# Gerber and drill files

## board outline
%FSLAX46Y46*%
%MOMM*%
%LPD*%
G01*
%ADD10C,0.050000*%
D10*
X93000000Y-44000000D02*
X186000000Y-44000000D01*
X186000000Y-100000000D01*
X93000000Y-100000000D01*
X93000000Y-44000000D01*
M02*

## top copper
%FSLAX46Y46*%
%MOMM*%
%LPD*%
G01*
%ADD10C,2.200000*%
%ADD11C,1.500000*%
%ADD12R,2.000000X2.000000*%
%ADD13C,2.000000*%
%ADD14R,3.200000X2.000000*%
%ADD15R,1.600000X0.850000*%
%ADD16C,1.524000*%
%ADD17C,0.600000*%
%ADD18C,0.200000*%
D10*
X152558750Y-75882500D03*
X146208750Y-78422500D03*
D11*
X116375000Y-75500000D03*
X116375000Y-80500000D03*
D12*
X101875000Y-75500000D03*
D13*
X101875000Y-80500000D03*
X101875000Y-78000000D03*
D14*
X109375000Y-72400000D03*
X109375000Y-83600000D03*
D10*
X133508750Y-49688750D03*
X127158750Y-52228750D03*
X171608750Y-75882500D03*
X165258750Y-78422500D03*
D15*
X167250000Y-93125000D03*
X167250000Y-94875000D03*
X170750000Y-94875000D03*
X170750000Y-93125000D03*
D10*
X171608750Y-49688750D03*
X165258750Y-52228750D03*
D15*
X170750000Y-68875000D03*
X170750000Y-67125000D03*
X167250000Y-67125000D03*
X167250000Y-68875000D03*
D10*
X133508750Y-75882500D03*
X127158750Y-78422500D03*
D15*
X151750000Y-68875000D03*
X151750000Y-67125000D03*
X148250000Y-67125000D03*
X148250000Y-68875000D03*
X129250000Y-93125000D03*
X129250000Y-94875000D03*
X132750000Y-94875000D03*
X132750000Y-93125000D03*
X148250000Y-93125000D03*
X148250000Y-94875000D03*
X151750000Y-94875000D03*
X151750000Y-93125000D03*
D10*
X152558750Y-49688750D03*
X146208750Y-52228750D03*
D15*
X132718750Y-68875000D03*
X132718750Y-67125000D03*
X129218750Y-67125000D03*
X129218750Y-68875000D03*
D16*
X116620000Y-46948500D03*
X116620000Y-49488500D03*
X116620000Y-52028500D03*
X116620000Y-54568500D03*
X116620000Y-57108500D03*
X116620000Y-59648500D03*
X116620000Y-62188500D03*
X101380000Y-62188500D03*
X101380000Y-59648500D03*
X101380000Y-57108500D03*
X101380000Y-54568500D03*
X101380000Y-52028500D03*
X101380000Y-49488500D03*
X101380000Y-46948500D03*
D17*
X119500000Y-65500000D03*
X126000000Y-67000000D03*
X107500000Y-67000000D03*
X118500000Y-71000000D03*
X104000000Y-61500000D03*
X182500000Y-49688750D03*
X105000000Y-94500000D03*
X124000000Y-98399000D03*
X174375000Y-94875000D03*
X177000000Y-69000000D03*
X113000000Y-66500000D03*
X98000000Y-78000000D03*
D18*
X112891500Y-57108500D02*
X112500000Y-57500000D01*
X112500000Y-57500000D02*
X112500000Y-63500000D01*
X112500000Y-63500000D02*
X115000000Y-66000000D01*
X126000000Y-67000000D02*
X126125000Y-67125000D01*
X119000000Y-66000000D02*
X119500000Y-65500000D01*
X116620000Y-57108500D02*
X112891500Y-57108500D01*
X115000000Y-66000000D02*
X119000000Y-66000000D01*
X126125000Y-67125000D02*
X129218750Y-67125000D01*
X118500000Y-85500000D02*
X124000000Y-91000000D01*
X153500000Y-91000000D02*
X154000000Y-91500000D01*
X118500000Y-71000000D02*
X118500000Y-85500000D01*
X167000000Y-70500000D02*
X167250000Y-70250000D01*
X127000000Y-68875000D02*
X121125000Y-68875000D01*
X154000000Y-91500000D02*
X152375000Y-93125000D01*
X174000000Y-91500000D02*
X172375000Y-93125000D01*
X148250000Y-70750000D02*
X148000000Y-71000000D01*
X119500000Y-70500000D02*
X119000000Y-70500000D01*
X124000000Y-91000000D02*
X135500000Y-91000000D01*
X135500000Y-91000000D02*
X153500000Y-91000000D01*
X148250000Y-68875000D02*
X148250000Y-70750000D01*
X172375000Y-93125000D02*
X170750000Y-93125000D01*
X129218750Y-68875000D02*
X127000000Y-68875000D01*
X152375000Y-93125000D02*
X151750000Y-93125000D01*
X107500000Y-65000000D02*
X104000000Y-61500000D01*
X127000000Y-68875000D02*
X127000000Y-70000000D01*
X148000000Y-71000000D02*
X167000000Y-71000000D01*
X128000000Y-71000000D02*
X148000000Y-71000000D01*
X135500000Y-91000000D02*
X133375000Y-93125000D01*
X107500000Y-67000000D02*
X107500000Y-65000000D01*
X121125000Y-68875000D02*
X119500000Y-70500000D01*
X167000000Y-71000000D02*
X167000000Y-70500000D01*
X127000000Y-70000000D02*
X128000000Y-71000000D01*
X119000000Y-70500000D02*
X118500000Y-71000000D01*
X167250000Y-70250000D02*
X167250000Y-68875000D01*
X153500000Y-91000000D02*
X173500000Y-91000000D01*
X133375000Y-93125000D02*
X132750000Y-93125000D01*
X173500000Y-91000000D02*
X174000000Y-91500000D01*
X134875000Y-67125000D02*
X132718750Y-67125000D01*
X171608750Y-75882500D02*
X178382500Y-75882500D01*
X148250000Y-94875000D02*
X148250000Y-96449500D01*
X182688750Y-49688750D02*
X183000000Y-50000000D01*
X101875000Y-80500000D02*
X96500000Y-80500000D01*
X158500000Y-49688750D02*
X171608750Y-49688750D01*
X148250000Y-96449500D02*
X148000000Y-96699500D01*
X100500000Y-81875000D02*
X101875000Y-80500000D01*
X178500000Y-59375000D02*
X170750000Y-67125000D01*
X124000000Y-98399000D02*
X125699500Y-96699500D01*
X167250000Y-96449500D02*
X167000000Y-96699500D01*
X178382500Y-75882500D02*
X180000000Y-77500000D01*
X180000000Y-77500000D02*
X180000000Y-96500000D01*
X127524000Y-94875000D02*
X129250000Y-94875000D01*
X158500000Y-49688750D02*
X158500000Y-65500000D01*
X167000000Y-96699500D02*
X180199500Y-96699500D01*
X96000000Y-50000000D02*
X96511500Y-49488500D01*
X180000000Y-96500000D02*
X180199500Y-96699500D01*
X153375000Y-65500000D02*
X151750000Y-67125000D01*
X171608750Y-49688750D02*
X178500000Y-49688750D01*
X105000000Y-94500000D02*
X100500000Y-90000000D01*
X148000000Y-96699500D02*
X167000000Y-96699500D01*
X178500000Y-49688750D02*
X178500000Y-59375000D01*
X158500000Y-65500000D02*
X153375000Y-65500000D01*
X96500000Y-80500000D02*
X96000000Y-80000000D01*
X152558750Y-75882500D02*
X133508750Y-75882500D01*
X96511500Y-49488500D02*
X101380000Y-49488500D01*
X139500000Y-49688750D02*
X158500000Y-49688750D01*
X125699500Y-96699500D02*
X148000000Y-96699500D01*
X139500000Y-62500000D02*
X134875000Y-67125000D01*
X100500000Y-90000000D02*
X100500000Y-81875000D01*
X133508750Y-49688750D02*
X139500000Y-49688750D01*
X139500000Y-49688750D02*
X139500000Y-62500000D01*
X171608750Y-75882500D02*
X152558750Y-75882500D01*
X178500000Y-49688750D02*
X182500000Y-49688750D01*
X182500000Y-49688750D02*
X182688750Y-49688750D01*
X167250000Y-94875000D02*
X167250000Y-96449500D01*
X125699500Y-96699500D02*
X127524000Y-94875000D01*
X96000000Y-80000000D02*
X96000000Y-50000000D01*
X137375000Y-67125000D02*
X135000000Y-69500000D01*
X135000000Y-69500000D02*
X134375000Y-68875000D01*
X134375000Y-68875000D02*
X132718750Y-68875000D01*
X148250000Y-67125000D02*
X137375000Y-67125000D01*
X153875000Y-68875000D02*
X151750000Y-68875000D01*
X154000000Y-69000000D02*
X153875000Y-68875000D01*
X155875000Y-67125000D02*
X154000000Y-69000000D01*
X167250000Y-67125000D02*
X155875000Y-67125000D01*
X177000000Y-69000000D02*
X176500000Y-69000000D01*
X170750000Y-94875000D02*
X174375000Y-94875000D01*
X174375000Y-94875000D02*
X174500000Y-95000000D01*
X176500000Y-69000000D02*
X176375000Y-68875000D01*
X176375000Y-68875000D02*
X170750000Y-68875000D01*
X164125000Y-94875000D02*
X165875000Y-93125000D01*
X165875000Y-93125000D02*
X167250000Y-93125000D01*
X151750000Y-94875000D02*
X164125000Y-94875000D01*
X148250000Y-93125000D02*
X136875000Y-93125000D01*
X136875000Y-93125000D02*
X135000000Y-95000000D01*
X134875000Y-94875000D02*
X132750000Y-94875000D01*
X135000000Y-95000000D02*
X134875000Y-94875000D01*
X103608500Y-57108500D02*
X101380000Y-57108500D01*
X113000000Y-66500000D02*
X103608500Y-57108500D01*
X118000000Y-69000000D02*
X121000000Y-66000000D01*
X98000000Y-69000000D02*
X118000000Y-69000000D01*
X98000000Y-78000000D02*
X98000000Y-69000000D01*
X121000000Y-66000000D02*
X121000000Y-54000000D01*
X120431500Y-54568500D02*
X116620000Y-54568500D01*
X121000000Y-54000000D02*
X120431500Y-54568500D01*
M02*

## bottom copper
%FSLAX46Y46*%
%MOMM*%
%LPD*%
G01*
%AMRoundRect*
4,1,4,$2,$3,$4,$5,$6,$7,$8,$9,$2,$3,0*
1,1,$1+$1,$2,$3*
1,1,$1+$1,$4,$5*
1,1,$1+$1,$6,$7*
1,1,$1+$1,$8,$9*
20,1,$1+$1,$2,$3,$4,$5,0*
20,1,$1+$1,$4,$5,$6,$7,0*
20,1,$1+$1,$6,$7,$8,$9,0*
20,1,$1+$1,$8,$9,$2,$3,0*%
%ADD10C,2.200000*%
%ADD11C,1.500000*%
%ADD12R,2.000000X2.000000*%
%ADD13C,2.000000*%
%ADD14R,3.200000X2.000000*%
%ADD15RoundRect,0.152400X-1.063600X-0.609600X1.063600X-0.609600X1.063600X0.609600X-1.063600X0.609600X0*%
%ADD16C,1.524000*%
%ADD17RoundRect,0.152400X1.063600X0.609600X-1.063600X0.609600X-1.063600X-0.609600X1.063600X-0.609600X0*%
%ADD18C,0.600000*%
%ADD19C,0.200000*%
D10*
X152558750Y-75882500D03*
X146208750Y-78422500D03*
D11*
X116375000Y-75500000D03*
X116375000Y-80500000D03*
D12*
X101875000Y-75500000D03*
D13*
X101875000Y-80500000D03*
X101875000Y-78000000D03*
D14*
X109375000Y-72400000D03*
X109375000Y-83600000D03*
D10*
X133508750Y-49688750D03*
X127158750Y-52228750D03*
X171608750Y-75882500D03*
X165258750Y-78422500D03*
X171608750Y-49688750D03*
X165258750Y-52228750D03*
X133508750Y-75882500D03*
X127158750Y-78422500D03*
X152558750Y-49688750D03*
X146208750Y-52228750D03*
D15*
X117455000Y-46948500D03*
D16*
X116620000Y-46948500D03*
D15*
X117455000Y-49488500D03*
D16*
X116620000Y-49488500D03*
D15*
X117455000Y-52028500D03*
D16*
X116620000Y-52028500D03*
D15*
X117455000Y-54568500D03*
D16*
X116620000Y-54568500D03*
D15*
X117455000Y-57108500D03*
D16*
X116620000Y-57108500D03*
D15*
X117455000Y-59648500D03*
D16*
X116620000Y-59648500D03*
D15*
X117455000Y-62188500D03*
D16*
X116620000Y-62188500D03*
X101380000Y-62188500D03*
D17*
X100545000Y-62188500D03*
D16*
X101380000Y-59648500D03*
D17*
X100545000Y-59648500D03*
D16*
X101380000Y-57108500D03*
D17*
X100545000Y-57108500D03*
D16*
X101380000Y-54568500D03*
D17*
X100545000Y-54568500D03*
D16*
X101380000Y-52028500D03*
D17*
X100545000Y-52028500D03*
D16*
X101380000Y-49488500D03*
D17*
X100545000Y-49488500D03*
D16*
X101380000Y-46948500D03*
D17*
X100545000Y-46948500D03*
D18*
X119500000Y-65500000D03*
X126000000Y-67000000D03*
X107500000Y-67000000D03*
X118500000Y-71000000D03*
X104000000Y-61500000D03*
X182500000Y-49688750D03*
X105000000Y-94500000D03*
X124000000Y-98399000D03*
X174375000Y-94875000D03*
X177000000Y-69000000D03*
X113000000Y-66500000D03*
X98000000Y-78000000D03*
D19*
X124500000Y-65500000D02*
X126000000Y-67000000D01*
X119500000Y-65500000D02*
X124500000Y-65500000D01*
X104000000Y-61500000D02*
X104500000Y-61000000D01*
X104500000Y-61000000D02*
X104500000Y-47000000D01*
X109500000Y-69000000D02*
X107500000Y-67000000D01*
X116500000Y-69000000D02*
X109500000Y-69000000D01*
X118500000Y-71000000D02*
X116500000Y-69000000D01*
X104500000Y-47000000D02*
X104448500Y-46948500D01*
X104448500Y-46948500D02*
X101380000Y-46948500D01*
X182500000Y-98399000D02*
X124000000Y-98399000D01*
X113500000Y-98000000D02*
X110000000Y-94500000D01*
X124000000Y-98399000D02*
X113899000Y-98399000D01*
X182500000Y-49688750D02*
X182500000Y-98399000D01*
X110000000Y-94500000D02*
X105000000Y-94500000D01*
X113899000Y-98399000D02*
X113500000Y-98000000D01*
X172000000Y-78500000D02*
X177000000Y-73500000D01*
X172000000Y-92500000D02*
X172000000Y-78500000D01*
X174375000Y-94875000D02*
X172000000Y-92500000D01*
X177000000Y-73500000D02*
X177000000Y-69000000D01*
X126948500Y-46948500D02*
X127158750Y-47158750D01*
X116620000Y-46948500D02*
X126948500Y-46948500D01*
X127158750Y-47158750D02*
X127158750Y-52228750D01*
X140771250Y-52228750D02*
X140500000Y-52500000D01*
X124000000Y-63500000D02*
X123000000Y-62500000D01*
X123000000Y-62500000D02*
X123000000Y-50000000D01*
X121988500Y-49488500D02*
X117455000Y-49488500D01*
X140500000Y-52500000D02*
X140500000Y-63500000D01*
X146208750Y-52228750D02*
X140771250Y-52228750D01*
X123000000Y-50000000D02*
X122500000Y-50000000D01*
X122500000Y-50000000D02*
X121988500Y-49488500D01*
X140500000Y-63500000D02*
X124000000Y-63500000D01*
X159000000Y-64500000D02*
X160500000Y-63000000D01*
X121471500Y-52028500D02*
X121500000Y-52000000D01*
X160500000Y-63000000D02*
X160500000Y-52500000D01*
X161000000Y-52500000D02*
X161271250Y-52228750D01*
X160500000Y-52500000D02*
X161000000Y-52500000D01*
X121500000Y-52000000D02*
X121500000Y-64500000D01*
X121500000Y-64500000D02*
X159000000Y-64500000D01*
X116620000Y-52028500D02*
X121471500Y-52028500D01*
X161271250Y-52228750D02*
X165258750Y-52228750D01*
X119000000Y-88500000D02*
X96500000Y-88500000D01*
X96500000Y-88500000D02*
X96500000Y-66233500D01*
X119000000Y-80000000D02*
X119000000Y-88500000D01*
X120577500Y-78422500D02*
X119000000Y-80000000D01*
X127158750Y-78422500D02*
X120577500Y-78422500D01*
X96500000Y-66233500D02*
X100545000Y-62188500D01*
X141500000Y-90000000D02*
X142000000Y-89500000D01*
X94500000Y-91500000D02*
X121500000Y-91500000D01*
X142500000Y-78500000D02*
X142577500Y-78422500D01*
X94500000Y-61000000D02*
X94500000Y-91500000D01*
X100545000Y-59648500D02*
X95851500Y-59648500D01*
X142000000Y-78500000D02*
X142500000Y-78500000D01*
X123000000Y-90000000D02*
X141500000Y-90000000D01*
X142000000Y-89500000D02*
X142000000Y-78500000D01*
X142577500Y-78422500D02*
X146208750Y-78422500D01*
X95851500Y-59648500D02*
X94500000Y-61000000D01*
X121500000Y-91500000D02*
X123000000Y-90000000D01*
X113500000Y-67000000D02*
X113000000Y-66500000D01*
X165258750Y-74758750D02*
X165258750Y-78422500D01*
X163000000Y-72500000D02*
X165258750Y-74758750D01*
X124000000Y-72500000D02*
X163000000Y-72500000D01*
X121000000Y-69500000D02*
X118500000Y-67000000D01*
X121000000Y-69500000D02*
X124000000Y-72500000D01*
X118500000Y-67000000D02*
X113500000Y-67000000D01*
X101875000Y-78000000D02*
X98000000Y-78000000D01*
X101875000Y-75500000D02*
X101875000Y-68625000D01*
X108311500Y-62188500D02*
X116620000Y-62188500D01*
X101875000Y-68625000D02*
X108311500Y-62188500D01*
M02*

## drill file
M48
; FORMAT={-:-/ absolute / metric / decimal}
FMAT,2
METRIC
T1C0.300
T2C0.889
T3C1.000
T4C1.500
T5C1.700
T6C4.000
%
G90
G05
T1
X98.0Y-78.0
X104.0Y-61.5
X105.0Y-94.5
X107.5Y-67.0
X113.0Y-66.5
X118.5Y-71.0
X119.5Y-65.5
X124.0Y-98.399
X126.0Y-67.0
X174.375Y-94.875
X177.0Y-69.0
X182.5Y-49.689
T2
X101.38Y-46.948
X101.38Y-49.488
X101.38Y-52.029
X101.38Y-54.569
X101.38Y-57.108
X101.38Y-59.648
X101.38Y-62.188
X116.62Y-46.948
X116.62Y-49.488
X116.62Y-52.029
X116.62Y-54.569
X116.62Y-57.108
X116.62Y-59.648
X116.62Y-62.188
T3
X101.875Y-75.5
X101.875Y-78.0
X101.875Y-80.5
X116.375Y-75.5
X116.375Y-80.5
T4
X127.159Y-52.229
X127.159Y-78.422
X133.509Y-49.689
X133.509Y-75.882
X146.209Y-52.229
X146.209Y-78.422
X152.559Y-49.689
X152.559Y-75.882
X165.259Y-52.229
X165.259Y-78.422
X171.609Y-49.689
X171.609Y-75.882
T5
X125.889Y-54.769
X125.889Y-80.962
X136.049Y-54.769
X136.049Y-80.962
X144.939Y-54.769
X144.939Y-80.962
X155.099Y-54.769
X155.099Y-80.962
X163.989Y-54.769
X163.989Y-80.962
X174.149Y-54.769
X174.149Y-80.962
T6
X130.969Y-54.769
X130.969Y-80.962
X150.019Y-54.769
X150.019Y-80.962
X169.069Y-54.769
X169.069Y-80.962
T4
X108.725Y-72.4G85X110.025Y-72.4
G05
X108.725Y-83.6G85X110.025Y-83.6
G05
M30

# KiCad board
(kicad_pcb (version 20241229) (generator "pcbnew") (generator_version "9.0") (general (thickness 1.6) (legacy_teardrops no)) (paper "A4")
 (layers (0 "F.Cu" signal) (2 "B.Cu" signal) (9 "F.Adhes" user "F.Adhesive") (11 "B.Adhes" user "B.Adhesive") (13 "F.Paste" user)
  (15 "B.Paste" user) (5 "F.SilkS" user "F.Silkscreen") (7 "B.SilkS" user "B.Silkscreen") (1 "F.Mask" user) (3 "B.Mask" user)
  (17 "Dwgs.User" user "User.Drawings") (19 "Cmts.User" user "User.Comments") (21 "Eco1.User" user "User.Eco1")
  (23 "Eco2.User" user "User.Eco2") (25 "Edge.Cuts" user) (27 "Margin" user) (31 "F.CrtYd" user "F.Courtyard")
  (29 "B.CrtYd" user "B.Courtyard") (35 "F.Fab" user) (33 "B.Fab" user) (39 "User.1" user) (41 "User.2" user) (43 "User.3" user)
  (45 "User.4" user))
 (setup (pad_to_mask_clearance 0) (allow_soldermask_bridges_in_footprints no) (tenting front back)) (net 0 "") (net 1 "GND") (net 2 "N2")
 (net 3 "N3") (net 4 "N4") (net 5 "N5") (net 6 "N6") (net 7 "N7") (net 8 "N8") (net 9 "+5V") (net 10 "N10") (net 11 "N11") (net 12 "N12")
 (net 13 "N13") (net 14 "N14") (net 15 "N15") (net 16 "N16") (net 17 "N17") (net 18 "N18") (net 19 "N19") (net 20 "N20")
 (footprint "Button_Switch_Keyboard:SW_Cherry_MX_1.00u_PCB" (layer "F.Cu") (at 152.55875 75.8825)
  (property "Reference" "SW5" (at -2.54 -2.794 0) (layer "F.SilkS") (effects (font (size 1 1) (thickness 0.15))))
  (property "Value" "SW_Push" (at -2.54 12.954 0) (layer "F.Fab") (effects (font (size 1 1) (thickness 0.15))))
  (pad "" np_thru_hole circle (at -7.62 5.08) (size 1.7 1.7) (drill 1.7) (layers "*.Cu" "*.Mask"))
  (pad "" np_thru_hole circle (at -2.54 5.08) (size 4 4) (drill 4) (layers "*.Cu" "*.Mask"))
  (pad "" np_thru_hole circle (at 2.54 5.08) (size 1.7 1.7) (drill 1.7) (layers "*.Cu" "*.Mask"))
  (pad "1" thru_hole circle (at 0 0) (size 2.2 2.2) (drill 1.5) (layers "*.Cu" "*.Mask") (remove_unused_layers no) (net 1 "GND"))
  (pad "2" thru_hole circle (at -6.35 2.54) (size 2.2 2.2) (drill 1.5) (layers "*.Cu" "*.Mask") (remove_unused_layers no) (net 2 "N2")))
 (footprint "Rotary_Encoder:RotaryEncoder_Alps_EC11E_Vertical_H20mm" (layer "F.Cu") (at 101.875 75.5)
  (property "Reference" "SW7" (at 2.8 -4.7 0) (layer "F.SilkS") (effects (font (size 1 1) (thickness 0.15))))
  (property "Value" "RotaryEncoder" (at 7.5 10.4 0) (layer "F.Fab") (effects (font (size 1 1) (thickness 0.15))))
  (pad "" thru_hole circle (at 14.5 0) (size 1.5 1.5) (drill 1) (layers "*.Cu" "*.Mask") (remove_unused_layers no))
  (pad "" thru_hole circle (at 14.5 5) (size 1.5 1.5) (drill 1) (layers "*.Cu" "*.Mask") (remove_unused_layers no))
  (pad "A" thru_hole rect (at 0 0) (size 2 2) (drill 1) (layers "*.Cu" "*.Mask") (remove_unused_layers no) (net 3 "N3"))
  (pad "B" thru_hole circle (at 0 5) (size 2 2) (drill 1) (layers "*.Cu" "*.Mask") (remove_unused_layers no) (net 1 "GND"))
  (pad "C" thru_hole circle (at 0 2.5) (size 2 2) (drill 1) (layers "*.Cu" "*.Mask") (remove_unused_layers no) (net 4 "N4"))
  (pad "MP" thru_hole rect (at 7.5 -3.1) (size 3.2 2) (drill oval 2.8 1.5) (layers "*.Cu" "*.Mask") (remove_unused_layers no))
  (pad "MP" thru_hole rect (at 7.5 8.1) (size 3.2 2) (drill oval 2.8 1.5) (layers "*.Cu" "*.Mask") (remove_unused_layers no)))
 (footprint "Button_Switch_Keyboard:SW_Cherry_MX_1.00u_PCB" (layer "F.Cu") (at 133.50875 49.68875)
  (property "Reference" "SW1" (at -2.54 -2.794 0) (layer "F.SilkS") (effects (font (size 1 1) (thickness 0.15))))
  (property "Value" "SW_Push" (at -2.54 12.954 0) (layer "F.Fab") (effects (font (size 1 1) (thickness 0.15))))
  (pad "" np_thru_hole circle (at -7.62 5.08) (size 1.7 1.7) (drill 1.7) (layers "*.Cu" "*.Mask"))
  (pad "" np_thru_hole circle (at -2.54 5.08) (size 4 4) (drill 4) (layers "*.Cu" "*.Mask"))
  (pad "" np_thru_hole circle (at 2.54 5.08) (size 1.7 1.7) (drill 1.7) (layers "*.Cu" "*.Mask"))
  (pad "1" thru_hole circle (at 0 0) (size 2.2 2.2) (drill 1.5) (layers "*.Cu" "*.Mask") (remove_unused_layers no) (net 1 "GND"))
  (pad "2" thru_hole circle (at -6.35 2.54) (size 2.2 2.2) (drill 1.5) (layers "*.Cu" "*.Mask") (remove_unused_layers no) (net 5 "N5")))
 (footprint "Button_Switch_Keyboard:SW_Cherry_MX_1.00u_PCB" (layer "F.Cu") (at 171.60875 75.8825)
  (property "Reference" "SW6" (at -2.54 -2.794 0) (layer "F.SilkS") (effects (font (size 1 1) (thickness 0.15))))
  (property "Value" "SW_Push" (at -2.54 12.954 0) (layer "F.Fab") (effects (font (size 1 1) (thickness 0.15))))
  (pad "" np_thru_hole circle (at -7.62 5.08) (size 1.7 1.7) (drill 1.7) (layers "*.Cu" "*.Mask"))
  (pad "" np_thru_hole circle (at -2.54 5.08) (size 4 4) (drill 4) (layers "*.Cu" "*.Mask"))
  (pad "" np_thru_hole circle (at 2.54 5.08) (size 1.7 1.7) (drill 1.7) (layers "*.Cu" "*.Mask"))
  (pad "1" thru_hole circle (at 0 0) (size 2.2 2.2) (drill 1.5) (layers "*.Cu" "*.Mask") (remove_unused_layers no) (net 1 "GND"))
  (pad "2" thru_hole circle (at -6.35 2.54) (size 2.2 2.2) (drill 1.5) (layers "*.Cu" "*.Mask") (remove_unused_layers no) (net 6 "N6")))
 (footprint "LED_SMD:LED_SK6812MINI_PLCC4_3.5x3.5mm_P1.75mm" (layer "F.Cu") (at 169 94)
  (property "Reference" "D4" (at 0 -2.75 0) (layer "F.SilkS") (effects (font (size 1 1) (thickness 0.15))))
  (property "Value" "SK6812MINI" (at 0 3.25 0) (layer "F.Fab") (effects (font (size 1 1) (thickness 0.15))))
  (pad "1" smd rect (at -1.75 -0.875) (size 1.6 0.85) (layers "F.Cu" "F.Mask" "F.Paste") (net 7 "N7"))
  (pad "2" smd rect (at -1.75 0.875) (size 1.6 0.85) (layers "F.Cu" "F.Mask" "F.Paste") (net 1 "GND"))
  (pad "3" smd rect (at 1.75 0.875) (size 1.6 0.85) (layers "F.Cu" "F.Mask" "F.Paste") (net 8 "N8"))
  (pad "4" smd rect (at 1.75 -0.875) (size 1.6 0.85) (layers "F.Cu" "F.Mask" "F.Paste") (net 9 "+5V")))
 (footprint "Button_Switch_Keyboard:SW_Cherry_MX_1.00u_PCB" (layer "F.Cu") (at 171.60875 49.68875)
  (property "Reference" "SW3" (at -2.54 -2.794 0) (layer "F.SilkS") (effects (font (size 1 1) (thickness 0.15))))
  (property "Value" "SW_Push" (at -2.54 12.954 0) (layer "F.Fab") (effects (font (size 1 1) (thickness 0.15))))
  (pad "" np_thru_hole circle (at -7.62 5.08) (size 1.7 1.7) (drill 1.7) (layers "*.Cu" "*.Mask"))
  (pad "" np_thru_hole circle (at -2.54 5.08) (size 4 4) (drill 4) (layers "*.Cu" "*.Mask"))
  (pad "" np_thru_hole circle (at 2.54 5.08) (size 1.7 1.7) (drill 1.7) (layers "*.Cu" "*.Mask"))
  (pad "1" thru_hole circle (at 0 0) (size 2.2 2.2) (drill 1.5) (layers "*.Cu" "*.Mask") (remove_unused_layers no) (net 1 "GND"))
  (pad "2" thru_hole circle (at -6.35 2.54) (size 2.2 2.2) (drill 1.5) (layers "*.Cu" "*.Mask") (remove_unused_layers no) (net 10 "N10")))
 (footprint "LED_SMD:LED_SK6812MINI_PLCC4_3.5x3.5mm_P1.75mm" (layer "F.Cu") (at 169 68 180)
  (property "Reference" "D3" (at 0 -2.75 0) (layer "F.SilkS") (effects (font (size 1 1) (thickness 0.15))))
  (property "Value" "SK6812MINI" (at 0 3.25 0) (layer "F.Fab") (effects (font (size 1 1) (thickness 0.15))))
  (pad "1" smd rect (at -1.75 -0.875 180) (size 1.6 0.85) (layers "F.Cu" "F.Mask" "F.Paste") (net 8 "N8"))
  (pad "2" smd rect (at -1.75 0.875 180) (size 1.6 0.85) (layers "F.Cu" "F.Mask" "F.Paste") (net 1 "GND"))
  (pad "3" smd rect (at 1.75 0.875 180) (size 1.6 0.85) (layers "F.Cu" "F.Mask" "F.Paste") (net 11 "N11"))
  (pad "4" smd rect (at 1.75 -0.875 180) (size 1.6 0.85) (layers "F.Cu" "F.Mask" "F.Paste") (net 9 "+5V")))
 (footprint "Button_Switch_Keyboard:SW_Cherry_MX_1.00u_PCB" (layer "F.Cu") (at 133.50875 75.8825)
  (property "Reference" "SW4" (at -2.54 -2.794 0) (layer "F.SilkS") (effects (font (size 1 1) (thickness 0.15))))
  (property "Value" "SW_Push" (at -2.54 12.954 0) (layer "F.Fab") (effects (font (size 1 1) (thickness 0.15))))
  (pad "" np_thru_hole circle (at -7.62 5.08) (size 1.7 1.7) (drill 1.7) (layers "*.Cu" "*.Mask"))
  (pad "" np_thru_hole circle (at -2.54 5.08) (size 4 4) (drill 4) (layers "*.Cu" "*.Mask"))
  (pad "" np_thru_hole circle (at 2.54 5.08) (size 1.7 1.7) (drill 1.7) (layers "*.Cu" "*.Mask"))
  (pad "1" thru_hole circle (at 0 0) (size 2.2 2.2) (drill 1.5) (layers "*.Cu" "*.Mask") (remove_unused_layers no) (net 1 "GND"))
  (pad "2" thru_hole circle (at -6.35 2.54) (size 2.2 2.2) (drill 1.5) (layers "*.Cu" "*.Mask") (remove_unused_layers no) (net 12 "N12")))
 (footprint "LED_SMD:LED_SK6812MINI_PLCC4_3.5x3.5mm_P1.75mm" (layer "F.Cu") (at 150 68 180)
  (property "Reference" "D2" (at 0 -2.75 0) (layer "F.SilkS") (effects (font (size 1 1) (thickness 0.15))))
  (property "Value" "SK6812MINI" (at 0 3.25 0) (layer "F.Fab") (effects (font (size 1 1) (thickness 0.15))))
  (pad "1" smd rect (at -1.75 -0.875 180) (size 1.6 0.85) (layers "F.Cu" "F.Mask" "F.Paste") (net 11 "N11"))
  (pad "2" smd rect (at -1.75 0.875 180) (size 1.6 0.85) (layers "F.Cu" "F.Mask" "F.Paste") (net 1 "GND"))
  (pad "3" smd rect (at 1.75 0.875 180) (size 1.6 0.85) (layers "F.Cu" "F.Mask" "F.Paste") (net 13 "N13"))
  (pad "4" smd rect (at 1.75 -0.875 180) (size 1.6 0.85) (layers "F.Cu" "F.Mask" "F.Paste") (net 9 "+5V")))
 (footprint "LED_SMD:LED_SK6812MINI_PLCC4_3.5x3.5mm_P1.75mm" (layer "F.Cu") (at 131 94)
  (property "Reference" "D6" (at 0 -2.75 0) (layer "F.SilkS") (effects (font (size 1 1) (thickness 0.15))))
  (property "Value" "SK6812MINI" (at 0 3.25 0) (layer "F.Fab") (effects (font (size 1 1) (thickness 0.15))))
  (pad "1" smd rect (at -1.75 -0.875) (size 1.6 0.85) (layers "F.Cu" "F.Mask" "F.Paste") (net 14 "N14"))
  (pad "2" smd rect (at -1.75 0.875) (size 1.6 0.85) (layers "F.Cu" "F.Mask" "F.Paste") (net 1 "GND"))
  (pad "3" smd rect (at 1.75 0.875) (size 1.6 0.85) (layers "F.Cu" "F.Mask" "F.Paste") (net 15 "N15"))
  (pad "4" smd rect (at 1.75 -0.875) (size 1.6 0.85) (layers "F.Cu" "F.Mask" "F.Paste") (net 9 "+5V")))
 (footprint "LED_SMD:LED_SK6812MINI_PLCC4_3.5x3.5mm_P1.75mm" (layer "F.Cu") (at 150 94)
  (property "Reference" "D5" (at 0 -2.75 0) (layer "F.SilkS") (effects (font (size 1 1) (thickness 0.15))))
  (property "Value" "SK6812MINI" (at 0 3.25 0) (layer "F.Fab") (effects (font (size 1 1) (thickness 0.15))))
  (pad "1" smd rect (at -1.75 -0.875) (size 1.6 0.85) (layers "F.Cu" "F.Mask" "F.Paste") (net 15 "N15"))
  (pad "2" smd rect (at -1.75 0.875) (size 1.6 0.85) (layers "F.Cu" "F.Mask" "F.Paste") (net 1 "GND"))
  (pad "3" smd rect (at 1.75 0.875) (size 1.6 0.85) (layers "F.Cu" "F.Mask" "F.Paste") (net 7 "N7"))
  (pad "4" smd rect (at 1.75 -0.875) (size 1.6 0.85) (layers "F.Cu" "F.Mask" "F.Paste") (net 9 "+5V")))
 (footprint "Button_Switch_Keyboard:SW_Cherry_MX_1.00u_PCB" (layer "F.Cu") (at 152.55875 49.68875)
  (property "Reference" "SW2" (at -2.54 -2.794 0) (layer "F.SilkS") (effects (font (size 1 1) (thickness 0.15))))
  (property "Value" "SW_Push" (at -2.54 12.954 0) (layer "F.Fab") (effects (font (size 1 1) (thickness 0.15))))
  (pad "" np_thru_hole circle (at -7.62 5.08) (size 1.7 1.7) (drill 1.7) (layers "*.Cu" "*.Mask"))
  (pad "" np_thru_hole circle (at -2.54 5.08) (size 4 4) (drill 4) (layers "*.Cu" "*.Mask"))
  (pad "" np_thru_hole circle (at 2.54 5.08) (size 1.7 1.7) (drill 1.7) (layers "*.Cu" "*.Mask"))
  (pad "1" thru_hole circle (at 0 0) (size 2.2 2.2) (drill 1.5) (layers "*.Cu" "*.Mask") (remove_unused_layers no) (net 1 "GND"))
  (pad "2" thru_hole circle (at -6.35 2.54) (size 2.2 2.2) (drill 1.5) (layers "*.Cu" "*.Mask") (remove_unused_layers no) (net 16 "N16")))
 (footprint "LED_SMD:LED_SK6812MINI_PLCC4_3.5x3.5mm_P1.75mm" (layer "F.Cu") (at 130.96875 68 180)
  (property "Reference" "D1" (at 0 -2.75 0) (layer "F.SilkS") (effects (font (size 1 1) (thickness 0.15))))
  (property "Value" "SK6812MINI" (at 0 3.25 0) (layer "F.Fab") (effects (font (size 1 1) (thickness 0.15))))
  (pad "1" smd rect (at -1.75 -0.875 180) (size 1.6 0.85) (layers "F.Cu" "F.Mask" "F.Paste") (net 13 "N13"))
  (pad "2" smd rect (at -1.75 0.875 180) (size 1.6 0.85) (layers "F.Cu" "F.Mask" "F.Paste") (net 1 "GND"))
  (pad "3" smd rect (at 1.75 0.875 180) (size 1.6 0.85) (layers "F.Cu" "F.Mask" "F.Paste") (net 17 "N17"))
  (pad "4" smd rect (at 1.75 -0.875 180) (size 1.6 0.85) (layers "F.Cu" "F.Mask" "F.Paste") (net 9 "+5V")))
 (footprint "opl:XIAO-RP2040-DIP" (layer "B.Cu") (at 109 54.5685 180)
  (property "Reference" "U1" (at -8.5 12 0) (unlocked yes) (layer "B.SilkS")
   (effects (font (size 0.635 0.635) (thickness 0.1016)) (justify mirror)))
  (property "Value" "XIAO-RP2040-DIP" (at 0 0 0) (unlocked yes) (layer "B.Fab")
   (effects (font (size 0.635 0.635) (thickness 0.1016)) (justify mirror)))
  (pad "1" smd roundrect (at -8.455 7.62) (size 2.432 1.524) (layers "B.Cu" "B.Mask") (roundrect_rratio 0.1) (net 5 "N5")
   (thermal_bridge_angle 45))
  (pad "1" thru_hole circle (at -7.62 7.62) (size 1.524 1.524) (drill 0.889) (layers "*.Cu" "*.Mask") (remove_unused_layers no) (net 5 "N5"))
  (pad "2" smd roundrect (at -8.455 5.08) (size 2.432 1.524) (layers "B.Cu" "B.Mask") (roundrect_rratio 0.1) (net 16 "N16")
   (thermal_bridge_angle 45))
  (pad "2" thru_hole circle (at -7.62 5.08) (size 1.524 1.524) (drill 0.889) (layers "*.Cu" "*.Mask") (remove_unused_layers no)
   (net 16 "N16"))
  (pad "3" smd roundrect (at -8.455 2.54) (size 2.432 1.524) (layers "B.Cu" "B.Mask") (roundrect_rratio 0.1) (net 10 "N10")
   (thermal_bridge_angle 45))
  (pad "3" thru_hole circle (at -7.62 2.54) (size 1.524 1.524) (drill 0.889) (layers "*.Cu" "*.Mask") (remove_unused_layers no)
   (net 10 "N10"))
  (pad "4" smd roundrect (at -8.455 0) (size 2.432 1.524) (layers "B.Cu" "B.Mask") (roundrect_rratio 0.1) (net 4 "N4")
   (thermal_bridge_angle 45))
  (pad "4" thru_hole circle (at -7.62 0) (size 1.524 1.524) (drill 0.889) (layers "*.Cu" "*.Mask") (remove_unused_layers no) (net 4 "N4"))
  (pad "5" smd roundrect (at -8.455 -2.54) (size 2.432 1.524) (layers "B.Cu" "B.Mask") (roundrect_rratio 0.1) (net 17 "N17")
   (thermal_bridge_angle 45))
  (pad "5" thru_hole circle (at -7.62 -2.54) (size 1.524 1.524) (drill 0.889) (layers "*.Cu" "*.Mask") (remove_unused_layers no)
   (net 17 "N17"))
  (pad "6" smd roundrect (at -8.455 -5.08) (size 2.432 1.524) (layers "B.Cu" "B.Mask") (roundrect_rratio 0.1) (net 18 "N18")
   (thermal_bridge_angle 45))
  (pad "6" thru_hole circle (at -7.62 -5.08) (size 1.524 1.524) (drill 0.889) (layers "*.Cu" "*.Mask") (remove_unused_layers no)
   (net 18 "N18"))
  (pad "7" smd roundrect (at -8.455 -7.62) (size 2.432 1.524) (layers "B.Cu" "B.Mask") (roundrect_rratio 0.1) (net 3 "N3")
   (thermal_bridge_angle 45))
  (pad "7" thru_hole circle (at -7.62 -7.62) (size 1.524 1.524) (drill 0.889) (layers "*.Cu" "*.Mask") (remove_unused_layers no)
   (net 3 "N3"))
  (pad "8" thru_hole circle (at 7.62 -7.62 180) (size 1.524 1.524) (drill 0.889) (layers "*.Cu" "*.Mask") (remove_unused_layers no)
   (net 12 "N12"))
  (pad "8" smd roundrect (at 8.455 -7.62 180) (size 2.432 1.524) (layers "B.Cu" "B.Mask") (roundrect_rratio 0.1) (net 12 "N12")
   (thermal_bridge_angle 45))
  (pad "9" thru_hole circle (at 7.62 -5.08 180) (size 1.524 1.524) (drill 0.889) (layers "*.Cu" "*.Mask") (remove_unused_layers no)
   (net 2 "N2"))
  (pad "9" smd roundrect (at 8.455 -5.08 180) (size 2.432 1.524) (layers "B.Cu" "B.Mask") (roundrect_rratio 0.1) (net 2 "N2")
   (thermal_bridge_angle 45))
  (pad "10" thru_hole circle (at 7.62 -2.54 180) (size 1.524 1.524) (drill 0.889) (layers "*.Cu" "*.Mask") (remove_unused_layers no)
   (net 6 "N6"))
  (pad "10" smd roundrect (at 8.455 -2.54 180) (size 2.432 1.524) (layers "B.Cu" "B.Mask") (roundrect_rratio 0.1) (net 6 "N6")
   (thermal_bridge_angle 45))
  (pad "11" thru_hole circle (at 7.62 0 180) (size 1.524 1.524) (drill 0.889) (layers "*.Cu" "*.Mask") (remove_unused_layers no)
   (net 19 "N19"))
  (pad "11" smd roundrect (at 8.455 0 180) (size 2.432 1.524) (layers "B.Cu" "B.Mask") (roundrect_rratio 0.1) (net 19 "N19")
   (thermal_bridge_angle 45))
  (pad "12" thru_hole circle (at 7.62 2.54 180) (size 1.524 1.524) (drill 0.889) (layers "*.Cu" "*.Mask") (remove_unused_layers no)
   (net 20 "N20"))
  (pad "12" smd roundrect (at 8.455 2.54 180) (size 2.432 1.524) (layers "B.Cu" "B.Mask") (roundrect_rratio 0.1) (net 20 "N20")
   (thermal_bridge_angle 45))
  (pad "13" thru_hole circle (at 7.62 5.08 180) (size 1.524 1.524) (drill 0.889) (layers "*.Cu" "*.Mask") (remove_unused_layers no)
   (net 1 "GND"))
  (pad "13" smd roundrect (at 8.455 5.08 180) (size 2.432 1.524) (layers "B.Cu" "B.Mask") (roundrect_rratio 0.1) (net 1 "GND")
   (thermal_bridge_angle 45))
  (pad "14" thru_hole circle (at 7.62 7.62 180) (size 1.524 1.524) (drill 0.889) (layers "*.Cu" "*.Mask") (remove_unused_layers no)
   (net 9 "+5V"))
  (pad "14" smd roundrect (at 8.455 7.62 180) (size 2.432 1.524) (layers "B.Cu" "B.Mask") (roundrect_rratio 0.1) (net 9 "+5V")
   (thermal_bridge_angle 45)))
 (gr_rect (start 93 44) (end 186 100) (stroke (width 0.05) (type default)) (fill no) (layer "Edge.Cuts"))
 (segment (start 112.8915 57.1085) (end 112.5 57.5) (width 0.2) (layer "F.Cu") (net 17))
 (segment (start 112.5 57.5) (end 112.5 63.5) (width 0.2) (layer "F.Cu") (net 17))
 (segment (start 112.5 63.5) (end 115 66) (width 0.2) (layer "F.Cu") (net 17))
 (segment (start 126 67) (end 126.125 67.125) (width 0.2) (layer "F.Cu") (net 17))
 (segment (start 119 66) (end 119.5 65.5) (width 0.2) (layer "F.Cu") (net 17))
 (segment (start 116.62 57.1085) (end 112.8915 57.1085) (width 0.2) (layer "F.Cu") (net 17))
 (segment (start 115 66) (end 119 66) (width 0.2) (layer "F.Cu") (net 17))
 (segment (start 126.125 67.125) (end 129.21875 67.125) (width 0.2) (layer "F.Cu") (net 17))
 (via (at 119.5 65.5) (size 0.6) (drill 0.3) (layers "F.Cu" "B.Cu") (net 17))
 (via (at 126 67) (size 0.6) (drill 0.3) (layers "F.Cu" "B.Cu") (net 17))
 (segment (start 124.5 65.5) (end 126 67) (width 0.2) (layer "B.Cu") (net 17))
 (segment (start 119.5 65.5) (end 124.5 65.5) (width 0.2) (layer "B.Cu") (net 17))
 (segment (start 118.5 85.5) (end 124 91) (width 0.2) (layer "F.Cu") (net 9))
 (segment (start 153.5 91) (end 154 91.5) (width 0.2) (layer "F.Cu") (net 9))
 (segment (start 118.5 71) (end 118.5 85.5) (width 0.2) (layer "F.Cu") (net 9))
 (segment (start 167 70.5) (end 167.25 70.25) (width 0.2) (layer "F.Cu") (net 9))
 (segment (start 127 68.875) (end 121.125 68.875) (width 0.2) (layer "F.Cu") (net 9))
 (segment (start 154 91.5) (end 152.375 93.125) (width 0.2) (layer "F.Cu") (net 9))
 (segment (start 174 91.5) (end 172.375 93.125) (width 0.2) (layer "F.Cu") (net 9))
 (segment (start 148.25 70.75) (end 148 71) (width 0.2) (layer "F.Cu") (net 9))
 (segment (start 119.5 70.5) (end 119 70.5) (width 0.2) (layer "F.Cu") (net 9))
 (segment (start 124 91) (end 135.5 91) (width 0.2) (layer "F.Cu") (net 9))
 (segment (start 135.5 91) (end 153.5 91) (width 0.2) (layer "F.Cu") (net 9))
 (segment (start 148.25 68.875) (end 148.25 70.75) (width 0.2) (layer "F.Cu") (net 9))
 (segment (start 172.375 93.125) (end 170.75 93.125) (width 0.2) (layer "F.Cu") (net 9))
 (segment (start 129.21875 68.875) (end 127 68.875) (width 0.2) (layer "F.Cu") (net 9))
 (segment (start 152.375 93.125) (end 151.75 93.125) (width 0.2) (layer "F.Cu") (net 9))
 (segment (start 107.5 65) (end 104 61.5) (width 0.2) (layer "F.Cu") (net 9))
 (segment (start 127 68.875) (end 127 70) (width 0.2) (layer "F.Cu") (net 9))
 (segment (start 148 71) (end 167 71) (width 0.2) (layer "F.Cu") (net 9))
 (segment (start 128 71) (end 148 71) (width 0.2) (layer "F.Cu") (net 9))
 (segment (start 135.5 91) (end 133.375 93.125) (width 0.2) (layer "F.Cu") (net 9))
 (segment (start 107.5 67) (end 107.5 65) (width 0.2) (layer "F.Cu") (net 9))
 (segment (start 121.125 68.875) (end 119.5 70.5) (width 0.2) (layer "F.Cu") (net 9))
 (segment (start 167 71) (end 167 70.5) (width 0.2) (layer "F.Cu") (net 9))
 (segment (start 127 70) (end 128 71) (width 0.2) (layer "F.Cu") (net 9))
 (segment (start 119 70.5) (end 118.5 71) (width 0.2) (layer "F.Cu") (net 9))
 (segment (start 167.25 70.25) (end 167.25 68.875) (width 0.2) (layer "F.Cu") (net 9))
 (segment (start 153.5 91) (end 173.5 91) (width 0.2) (layer "F.Cu") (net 9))
 (segment (start 133.375 93.125) (end 132.75 93.125) (width 0.2) (layer "F.Cu") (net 9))
 (segment (start 173.5 91) (end 174 91.5) (width 0.2) (layer "F.Cu") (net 9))
 (via (at 107.5 67) (size 0.6) (drill 0.3) (layers "F.Cu" "B.Cu") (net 9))
 (via (at 118.5 71) (size 0.6) (drill 0.3) (layers "F.Cu" "B.Cu") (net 9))
 (via (at 104 61.5) (size 0.6) (drill 0.3) (layers "F.Cu" "B.Cu") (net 9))
 (segment (start 104 61.5) (end 104.5 61) (width 0.2) (layer "B.Cu") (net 9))
 (segment (start 104.5 61) (end 104.5 47) (width 0.2) (layer "B.Cu") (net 9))
 (segment (start 109.5 69) (end 107.5 67) (width 0.2) (layer "B.Cu") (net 9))
 (segment (start 116.5 69) (end 109.5 69) (width 0.2) (layer "B.Cu") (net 9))
 (segment (start 118.5 71) (end 116.5 69) (width 0.2) (layer "B.Cu") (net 9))
 (segment (start 104.5 47) (end 104.4485 46.9485) (width 0.2) (layer "B.Cu") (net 9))
 (segment (start 104.4485 46.9485) (end 101.38 46.9485) (width 0.2) (layer "B.Cu") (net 9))
 (segment (start 134.875 67.125) (end 132.71875 67.125) (width 0.2) (layer "F.Cu") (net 1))
 (segment (start 171.60875 75.8825) (end 178.3825 75.8825) (width 0.2) (layer "F.Cu") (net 1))
 (segment (start 148.25 94.875) (end 148.25 96.4495) (width 0.2) (layer "F.Cu") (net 1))
 (segment (start 182.68875 49.68875) (end 183 50) (width 0.2) (layer "F.Cu") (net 1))
 (segment (start 101.875 80.5) (end 96.5 80.5) (width 0.2) (layer "F.Cu") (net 1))
 (segment (start 158.5 49.68875) (end 171.60875 49.68875) (width 0.2) (layer "F.Cu") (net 1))
 (segment (start 148.25 96.4495) (end 148 96.6995) (width 0.2) (layer "F.Cu") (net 1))
 (segment (start 100.5 81.875) (end 101.875 80.5) (width 0.2) (layer "F.Cu") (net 1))
 (segment (start 178.5 59.375) (end 170.75 67.125) (width 0.2) (layer "F.Cu") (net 1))
 (segment (start 124 98.399) (end 125.6995 96.6995) (width 0.2) (layer "F.Cu") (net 1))
 (segment (start 167.25 96.4495) (end 167 96.6995) (width 0.2) (layer "F.Cu") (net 1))
 (segment (start 178.3825 75.8825) (end 180 77.5) (width 0.2) (layer "F.Cu") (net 1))
 (segment (start 180 77.5) (end 180 96.5) (width 0.2) (layer "F.Cu") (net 1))
 (segment (start 127.524 94.875) (end 129.25 94.875) (width 0.2) (layer "F.Cu") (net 1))
 (segment (start 158.5 49.68875) (end 158.5 65.5) (width 0.2) (layer "F.Cu") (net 1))
 (segment (start 167 96.6995) (end 180.1995 96.6995) (width 0.2) (layer "F.Cu") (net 1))
 (segment (start 96 50) (end 96.5115 49.4885) (width 0.2) (layer "F.Cu") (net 1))
 (segment (start 180 96.5) (end 180.1995 96.6995) (width 0.2) (layer "F.Cu") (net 1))
 (segment (start 153.375 65.5) (end 151.75 67.125) (width 0.2) (layer "F.Cu") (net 1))
 (segment (start 171.60875 49.68875) (end 178.5 49.68875) (width 0.2) (layer "F.Cu") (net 1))
 (segment (start 105 94.5) (end 100.5 90) (width 0.2) (layer "F.Cu") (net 1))
 (segment (start 148 96.6995) (end 167 96.6995) (width 0.2) (layer "F.Cu") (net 1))
 (segment (start 178.5 49.68875) (end 178.5 59.375) (width 0.2) (layer "F.Cu") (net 1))
 (segment (start 158.5 65.5) (end 153.375 65.5) (width 0.2) (layer "F.Cu") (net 1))
 (segment (start 96.5 80.5) (end 96 80) (width 0.2) (layer "F.Cu") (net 1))
 (segment (start 152.55875 75.8825) (end 133.50875 75.8825) (width 0.2) (layer "F.Cu") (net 1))
 (segment (start 96.5115 49.4885) (end 101.38 49.4885) (width 0.2) (layer "F.Cu") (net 1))
 (segment (start 139.5 49.68875) (end 158.5 49.68875) (width 0.2) (layer "F.Cu") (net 1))
 (segment (start 125.6995 96.6995) (end 148 96.6995) (width 0.2) (layer "F.Cu") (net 1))
 (segment (start 139.5 62.5) (end 134.875 67.125) (width 0.2) (layer "F.Cu") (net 1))
 (segment (start 100.5 90) (end 100.5 81.875) (width 0.2) (layer "F.Cu") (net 1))
 (segment (start 133.50875 49.68875) (end 139.5 49.68875) (width 0.2) (layer "F.Cu") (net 1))
 (segment (start 139.5 49.68875) (end 139.5 62.5) (width 0.2) (layer "F.Cu") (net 1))
 (segment (start 171.60875 75.8825) (end 152.55875 75.8825) (width 0.2) (layer "F.Cu") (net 1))
 (segment (start 178.5 49.68875) (end 182.5 49.68875) (width 0.2) (layer "F.Cu") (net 1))
 (segment (start 182.5 49.68875) (end 182.68875 49.68875) (width 0.2) (layer "F.Cu") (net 1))
 (segment (start 167.25 94.875) (end 167.25 96.4495) (width 0.2) (layer "F.Cu") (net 1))
 (segment (start 125.6995 96.6995) (end 127.524 94.875) (width 0.2) (layer "F.Cu") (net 1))
 (segment (start 96 80) (end 96 50) (width 0.2) (layer "F.Cu") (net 1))
 (via (at 182.5 49.68875) (size 0.6) (drill 0.3) (layers "F.Cu" "B.Cu") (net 1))
 (via (at 105 94.5) (size 0.6) (drill 0.3) (layers "F.Cu" "B.Cu") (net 1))
 (via (at 124 98.399) (size 0.6) (drill 0.3) (layers "F.Cu" "B.Cu") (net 1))
 (segment (start 182.5 98.399) (end 124 98.399) (width 0.2) (layer "B.Cu") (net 1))
 (segment (start 113.5 98) (end 110 94.5) (width 0.2) (layer "B.Cu") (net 1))
 (segment (start 124 98.399) (end 113.899 98.399) (width 0.2) (layer "B.Cu") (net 1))
 (segment (start 182.5 49.68875) (end 182.5 98.399) (width 0.2) (layer "B.Cu") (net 1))
 (segment (start 110 94.5) (end 105 94.5) (width 0.2) (layer "B.Cu") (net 1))
 (segment (start 113.899 98.399) (end 113.5 98) (width 0.2) (layer "B.Cu") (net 1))
 (segment (start 137.375 67.125) (end 135 69.5) (width 0.2) (layer "F.Cu") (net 13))
 (segment (start 135 69.5) (end 134.375 68.875) (width 0.2) (layer "F.Cu") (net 13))
 (segment (start 134.375 68.875) (end 132.71875 68.875) (width 0.2) (layer "F.Cu") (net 13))
 (segment (start 148.25 67.125) (end 137.375 67.125) (width 0.2) (layer "F.Cu") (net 13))
 (segment (start 153.875 68.875) (end 151.75 68.875) (width 0.2) (layer "F.Cu") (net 11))
 (segment (start 154 69) (end 153.875 68.875) (width 0.2) (layer "F.Cu") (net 11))
 (segment (start 155.875 67.125) (end 154 69) (width 0.2) (layer "F.Cu") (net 11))
 (segment (start 167.25 67.125) (end 155.875 67.125) (width 0.2) (layer "F.Cu") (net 11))
 (segment (start 177 69) (end 176.5 69) (width 0.2) (layer "F.Cu") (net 8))
 (segment (start 170.75 94.875) (end 174.375 94.875) (width 0.2) (layer "F.Cu") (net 8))
 (segment (start 174.375 94.875) (end 174.5 95) (width 0.2) (layer "F.Cu") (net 8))
 (segment (start 176.5 69) (end 176.375 68.875) (width 0.2) (layer "F.Cu") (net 8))
 (segment (start 176.375 68.875) (end 170.75 68.875) (width 0.2) (layer "F.Cu") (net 8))
 (via (at 174.375 94.875) (size 0.6) (drill 0.3) (layers "F.Cu" "B.Cu") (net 8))
 (via (at 177 69) (size 0.6) (drill 0.3) (layers "F.Cu" "B.Cu") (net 8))
 (segment (start 172 78.5) (end 177 73.5) (width 0.2) (layer "B.Cu") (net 8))
 (segment (start 172 92.5) (end 172 78.5) (width 0.2) (layer "B.Cu") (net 8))
 (segment (start 174.375 94.875) (end 172 92.5) (width 0.2) (layer "B.Cu") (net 8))
 (segment (start 177 73.5) (end 177 69) (width 0.2) (layer "B.Cu") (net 8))
 (segment (start 164.125 94.875) (end 165.875 93.125) (width 0.2) (layer "F.Cu") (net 7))
 (segment (start 165.875 93.125) (end 167.25 93.125) (width 0.2) (layer "F.Cu") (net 7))
 (segment (start 151.75 94.875) (end 164.125 94.875) (width 0.2) (layer "F.Cu") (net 7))
 (segment (start 148.25 93.125) (end 136.875 93.125) (width 0.2) (layer "F.Cu") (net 15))
 (segment (start 136.875 93.125) (end 135 95) (width 0.2) (layer "F.Cu") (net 15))
 (segment (start 134.875 94.875) (end 132.75 94.875) (width 0.2) (layer "F.Cu") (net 15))
 (segment (start 135 95) (end 134.875 94.875) (width 0.2) (layer "F.Cu") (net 15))
 (segment (start 126.9485 46.9485) (end 127.15875 47.15875) (width 0.2) (layer "B.Cu") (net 5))
 (segment (start 116.62 46.9485) (end 126.9485 46.9485) (width 0.2) (layer "B.Cu") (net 5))
 (segment (start 127.15875 47.15875) (end 127.15875 52.22875) (width 0.2) (layer "B.Cu") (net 5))
 (segment (start 140.77125 52.22875) (end 140.5 52.5) (width 0.2) (layer "B.Cu") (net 16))
 (segment (start 124 63.5) (end 123 62.5) (width 0.2) (layer "B.Cu") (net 16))
 (segment (start 123 62.5) (end 123 50) (width 0.2) (layer "B.Cu") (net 16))
 (segment (start 121.9885 49.4885) (end 117.455 49.4885) (width 0.2) (layer "B.Cu") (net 16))
 (segment (start 140.5 52.5) (end 140.5 63.5) (width 0.2) (layer "B.Cu") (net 16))
 (segment (start 146.20875 52.22875) (end 140.77125 52.22875) (width 0.2) (layer "B.Cu") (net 16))
 (segment (start 123 50) (end 122.5 50) (width 0.2) (layer "B.Cu") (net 16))
 (segment (start 122.5 50) (end 121.9885 49.4885) (width 0.2) (layer "B.Cu") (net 16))
 (segment (start 140.5 63.5) (end 124 63.5) (width 0.2) (layer "B.Cu") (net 16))
 (segment (start 159 64.5) (end 160.5 63) (width 0.2) (layer "B.Cu") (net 10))
 (segment (start 121.4715 52.0285) (end 121.5 52) (width 0.2) (layer "B.Cu") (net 10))
 (segment (start 160.5 63) (end 160.5 52.5) (width 0.2) (layer "B.Cu") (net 10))
 (segment (start 161 52.5) (end 161.27125 52.22875) (width 0.2) (layer "B.Cu") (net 10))
 (segment (start 160.5 52.5) (end 161 52.5) (width 0.2) (layer "B.Cu") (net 10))
 (segment (start 121.5 52) (end 121.5 64.5) (width 0.2) (layer "B.Cu") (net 10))
 (segment (start 121.5 64.5) (end 159 64.5) (width 0.2) (layer "B.Cu") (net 10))
 (segment (start 116.62 52.0285) (end 121.4715 52.0285) (width 0.2) (layer "B.Cu") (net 10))
 (segment (start 161.27125 52.22875) (end 165.25875 52.22875) (width 0.2) (layer "B.Cu") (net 10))
 (segment (start 119 88.5) (end 96.5 88.5) (width 0.2) (layer "B.Cu") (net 12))
 (segment (start 96.5 88.5) (end 96.5 66.2335) (width 0.2) (layer "B.Cu") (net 12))
 (segment (start 119 80) (end 119 88.5) (width 0.2) (layer "B.Cu") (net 12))
 (segment (start 120.5775 78.4225) (end 119 80) (width 0.2) (layer "B.Cu") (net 12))
 (segment (start 127.15875 78.4225) (end 120.5775 78.4225) (width 0.2) (layer "B.Cu") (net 12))
 (segment (start 96.5 66.2335) (end 100.545 62.1885) (width 0.2) (layer "B.Cu") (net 12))
 (segment (start 141.5 90) (end 142 89.5) (width 0.2) (layer "B.Cu") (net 2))
 (segment (start 94.5 91.5) (end 121.5 91.5) (width 0.2) (layer "B.Cu") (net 2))
 (segment (start 142.5 78.5) (end 142.5775 78.4225) (width 0.2) (layer "B.Cu") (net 2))
 (segment (start 94.5 61) (end 94.5 91.5) (width 0.2) (layer "B.Cu") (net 2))
 (segment (start 100.545 59.6485) (end 95.8515 59.6485) (width 0.2) (layer "B.Cu") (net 2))
 (segment (start 142 78.5) (end 142.5 78.5) (width 0.2) (layer "B.Cu") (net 2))
 (segment (start 123 90) (end 141.5 90) (width 0.2) (layer "B.Cu") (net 2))
 (segment (start 142 89.5) (end 142 78.5) (width 0.2) (layer "B.Cu") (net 2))
 (segment (start 142.5775 78.4225) (end 146.20875 78.4225) (width 0.2) (layer "B.Cu") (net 2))
 (segment (start 95.8515 59.6485) (end 94.5 61) (width 0.2) (layer "B.Cu") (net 2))
 (segment (start 121.5 91.5) (end 123 90) (width 0.2) (layer "B.Cu") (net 2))
 (segment (start 103.6085 57.1085) (end 101.38 57.1085) (width 0.2) (layer "F.Cu") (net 6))
 (segment (start 113 66.5) (end 103.6085 57.1085) (width 0.2) (layer "F.Cu") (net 6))
 (via (at 113 66.5) (size 0.6) (drill 0.3) (layers "F.Cu" "B.Cu") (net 6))
 (segment (start 113.5 67) (end 113 66.5) (width 0.2) (layer "B.Cu") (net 6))
 (segment (start 165.25875 74.75875) (end 165.25875 78.4225) (width 0.2) (layer "B.Cu") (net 6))
 (segment (start 163 72.5) (end 165.25875 74.75875) (width 0.2) (layer "B.Cu") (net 6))
 (segment (start 124 72.5) (end 163 72.5) (width 0.2) (layer "B.Cu") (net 6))
 (segment (start 121 69.5) (end 118.5 67) (width 0.2) (layer "B.Cu") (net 6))
 (segment (start 121 69.5) (end 124 72.5) (width 0.2) (layer "B.Cu") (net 6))
 (segment (start 118.5 67) (end 113.5 67) (width 0.2) (layer "B.Cu") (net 6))
 (segment (start 118 69) (end 121 66) (width 0.2) (layer "F.Cu") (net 4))
 (segment (start 98 69) (end 118 69) (width 0.2) (layer "F.Cu") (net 4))
 (segment (start 98 78) (end 98 69) (width 0.2) (layer "F.Cu") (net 4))
 (segment (start 121 66) (end 121 54) (width 0.2) (layer "F.Cu") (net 4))
 (segment (start 120.4315 54.5685) (end 116.62 54.5685) (width 0.2) (layer "F.Cu") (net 4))
 (segment (start 121 54) (end 120.4315 54.5685) (width 0.2) (layer "F.Cu") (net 4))
 (via (at 98 78) (size 0.6) (drill 0.3) (layers "F.Cu" "B.Cu") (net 4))
 (segment (start 101.875 78) (end 98 78) (width 0.2) (layer "B.Cu") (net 4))
 (segment (start 101.875 75.5) (end 101.875 68.625) (width 0.2) (layer "B.Cu") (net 3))
 (segment (start 108.3115 62.1885) (end 116.62 62.1885) (width 0.2) (layer "B.Cu") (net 3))
 (segment (start 101.875 68.625) (end 108.3115 62.1885) (width 0.2) (layer "B.Cu") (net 3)))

